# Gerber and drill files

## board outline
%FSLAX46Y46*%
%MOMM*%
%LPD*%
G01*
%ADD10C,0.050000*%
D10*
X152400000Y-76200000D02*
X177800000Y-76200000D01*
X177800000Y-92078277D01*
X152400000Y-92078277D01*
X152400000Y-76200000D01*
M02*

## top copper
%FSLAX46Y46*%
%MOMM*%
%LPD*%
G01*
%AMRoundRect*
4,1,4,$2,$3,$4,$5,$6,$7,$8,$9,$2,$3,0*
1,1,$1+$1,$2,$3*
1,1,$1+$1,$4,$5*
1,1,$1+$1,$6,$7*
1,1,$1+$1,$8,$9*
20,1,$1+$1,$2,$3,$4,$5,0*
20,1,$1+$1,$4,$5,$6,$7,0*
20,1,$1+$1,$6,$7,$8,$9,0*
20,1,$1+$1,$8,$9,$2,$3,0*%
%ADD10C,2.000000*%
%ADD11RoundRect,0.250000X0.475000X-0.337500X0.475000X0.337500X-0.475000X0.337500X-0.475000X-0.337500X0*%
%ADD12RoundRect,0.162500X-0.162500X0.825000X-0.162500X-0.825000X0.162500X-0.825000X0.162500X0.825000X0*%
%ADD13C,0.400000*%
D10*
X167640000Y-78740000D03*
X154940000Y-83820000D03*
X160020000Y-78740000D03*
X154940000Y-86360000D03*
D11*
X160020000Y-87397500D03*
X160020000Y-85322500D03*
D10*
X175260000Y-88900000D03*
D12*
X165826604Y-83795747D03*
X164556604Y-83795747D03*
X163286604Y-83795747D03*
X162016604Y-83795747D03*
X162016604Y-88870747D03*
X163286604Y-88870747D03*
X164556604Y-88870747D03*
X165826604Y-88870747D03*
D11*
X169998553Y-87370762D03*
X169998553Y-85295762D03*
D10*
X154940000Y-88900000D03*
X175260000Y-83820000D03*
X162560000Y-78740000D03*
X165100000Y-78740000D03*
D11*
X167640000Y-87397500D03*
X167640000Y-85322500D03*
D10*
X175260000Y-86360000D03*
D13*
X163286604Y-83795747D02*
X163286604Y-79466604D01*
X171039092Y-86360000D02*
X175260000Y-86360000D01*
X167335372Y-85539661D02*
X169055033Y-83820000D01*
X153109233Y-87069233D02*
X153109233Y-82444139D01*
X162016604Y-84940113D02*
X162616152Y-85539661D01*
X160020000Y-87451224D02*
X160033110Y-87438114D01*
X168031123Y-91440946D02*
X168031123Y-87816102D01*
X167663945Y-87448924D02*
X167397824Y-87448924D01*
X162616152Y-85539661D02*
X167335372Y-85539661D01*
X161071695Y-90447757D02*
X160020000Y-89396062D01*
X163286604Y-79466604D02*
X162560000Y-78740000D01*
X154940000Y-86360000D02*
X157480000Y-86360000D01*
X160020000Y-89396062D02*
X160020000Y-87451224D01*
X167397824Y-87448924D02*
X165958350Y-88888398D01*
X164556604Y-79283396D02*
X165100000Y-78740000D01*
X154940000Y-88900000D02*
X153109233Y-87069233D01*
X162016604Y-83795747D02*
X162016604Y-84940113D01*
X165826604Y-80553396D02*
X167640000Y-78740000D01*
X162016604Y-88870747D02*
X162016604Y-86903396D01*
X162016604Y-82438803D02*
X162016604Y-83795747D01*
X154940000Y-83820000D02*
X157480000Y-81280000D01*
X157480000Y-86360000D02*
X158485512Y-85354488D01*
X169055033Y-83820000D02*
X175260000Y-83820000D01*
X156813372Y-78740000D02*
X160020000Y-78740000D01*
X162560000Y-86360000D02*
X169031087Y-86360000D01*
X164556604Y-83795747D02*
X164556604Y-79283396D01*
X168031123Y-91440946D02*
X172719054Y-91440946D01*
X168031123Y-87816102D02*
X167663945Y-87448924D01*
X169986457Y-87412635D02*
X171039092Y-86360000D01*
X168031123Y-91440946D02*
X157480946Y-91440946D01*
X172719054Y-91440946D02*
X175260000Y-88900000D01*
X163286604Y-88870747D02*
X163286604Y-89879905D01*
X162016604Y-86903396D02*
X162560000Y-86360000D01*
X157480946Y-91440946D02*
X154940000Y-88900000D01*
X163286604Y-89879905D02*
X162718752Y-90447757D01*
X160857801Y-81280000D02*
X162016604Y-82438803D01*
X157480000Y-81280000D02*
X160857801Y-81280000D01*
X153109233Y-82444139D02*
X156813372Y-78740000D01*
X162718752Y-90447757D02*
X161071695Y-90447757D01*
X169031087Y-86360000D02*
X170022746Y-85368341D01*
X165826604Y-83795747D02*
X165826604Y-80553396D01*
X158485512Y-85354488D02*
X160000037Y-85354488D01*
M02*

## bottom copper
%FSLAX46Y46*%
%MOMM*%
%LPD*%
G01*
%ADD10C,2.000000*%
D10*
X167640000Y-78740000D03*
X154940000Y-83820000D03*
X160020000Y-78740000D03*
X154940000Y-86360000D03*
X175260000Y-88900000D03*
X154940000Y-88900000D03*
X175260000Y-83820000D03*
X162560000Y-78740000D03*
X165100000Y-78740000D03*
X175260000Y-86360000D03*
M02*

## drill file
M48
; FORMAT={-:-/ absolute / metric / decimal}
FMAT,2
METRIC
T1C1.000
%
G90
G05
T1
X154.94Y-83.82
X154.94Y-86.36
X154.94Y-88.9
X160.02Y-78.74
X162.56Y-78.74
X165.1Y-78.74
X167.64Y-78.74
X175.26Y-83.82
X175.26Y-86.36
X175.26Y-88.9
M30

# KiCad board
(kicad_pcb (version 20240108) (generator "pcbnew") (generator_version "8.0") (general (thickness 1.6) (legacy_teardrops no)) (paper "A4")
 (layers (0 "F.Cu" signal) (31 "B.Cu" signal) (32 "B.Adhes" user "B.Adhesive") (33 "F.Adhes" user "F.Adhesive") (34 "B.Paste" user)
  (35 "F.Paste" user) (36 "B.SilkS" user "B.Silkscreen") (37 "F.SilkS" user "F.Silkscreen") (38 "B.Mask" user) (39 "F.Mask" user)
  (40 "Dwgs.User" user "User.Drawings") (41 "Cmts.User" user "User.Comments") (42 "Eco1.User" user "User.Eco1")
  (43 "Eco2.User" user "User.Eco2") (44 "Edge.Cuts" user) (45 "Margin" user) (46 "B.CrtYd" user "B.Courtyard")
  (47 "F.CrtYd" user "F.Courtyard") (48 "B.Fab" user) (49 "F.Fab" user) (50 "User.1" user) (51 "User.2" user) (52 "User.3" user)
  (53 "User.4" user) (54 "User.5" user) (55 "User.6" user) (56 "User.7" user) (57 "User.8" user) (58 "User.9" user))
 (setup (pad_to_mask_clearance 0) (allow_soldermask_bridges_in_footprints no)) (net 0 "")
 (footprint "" (layer "F.Cu") (at 167.64 78.74)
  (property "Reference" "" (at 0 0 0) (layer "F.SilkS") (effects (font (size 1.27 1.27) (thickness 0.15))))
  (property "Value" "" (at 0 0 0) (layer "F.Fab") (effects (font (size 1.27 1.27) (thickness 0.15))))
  (pad "1" thru_hole circle (at 0 0) (size 2 2) (drill 1) (layers "*.Cu" "*.Mask") (remove_unused_layers no)))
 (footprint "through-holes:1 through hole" (layer "F.Cu") (at 154.94 83.82)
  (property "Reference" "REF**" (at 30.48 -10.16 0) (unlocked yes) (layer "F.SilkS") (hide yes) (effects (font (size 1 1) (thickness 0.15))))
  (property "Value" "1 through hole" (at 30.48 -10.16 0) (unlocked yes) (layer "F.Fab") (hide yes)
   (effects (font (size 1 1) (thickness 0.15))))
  (pad "1" thru_hole circle (at 0 0) (size 2 2) (drill 1) (layers "*.Cu" "*.Mask") (remove_unused_layers no)))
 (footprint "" (layer "F.Cu") (at 160.02 78.74)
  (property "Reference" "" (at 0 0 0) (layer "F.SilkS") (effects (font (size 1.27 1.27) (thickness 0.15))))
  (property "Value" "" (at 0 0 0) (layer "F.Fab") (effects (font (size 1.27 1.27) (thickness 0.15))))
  (pad "1" thru_hole circle (at 0 0) (size 2 2) (drill 1) (layers "*.Cu" "*.Mask") (remove_unused_layers no)))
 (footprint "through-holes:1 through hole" (layer "F.Cu") (at 154.94 86.36)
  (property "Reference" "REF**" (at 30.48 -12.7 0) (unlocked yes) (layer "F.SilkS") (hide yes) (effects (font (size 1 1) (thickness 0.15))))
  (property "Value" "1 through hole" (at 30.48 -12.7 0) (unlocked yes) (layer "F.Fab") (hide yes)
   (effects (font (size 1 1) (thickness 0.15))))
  (pad "1" thru_hole circle (at 0 0) (size 2 2) (drill 1) (layers "*.Cu" "*.Mask") (remove_unused_layers no)))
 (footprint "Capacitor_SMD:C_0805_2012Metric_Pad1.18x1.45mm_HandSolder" (layer "F.Cu") (at 160.02 86.36 90)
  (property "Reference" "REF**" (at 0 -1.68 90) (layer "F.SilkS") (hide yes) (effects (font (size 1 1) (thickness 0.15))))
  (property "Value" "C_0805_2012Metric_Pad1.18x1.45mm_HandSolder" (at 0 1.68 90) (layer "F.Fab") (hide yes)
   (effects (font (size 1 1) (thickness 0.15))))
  (pad "1" smd roundrect (at -1.0375 0 90) (size 1.175 1.45) (layers "F.Cu" "F.Paste" "F.Mask") (roundrect_rratio 0.212766))
  (pad "2" smd roundrect (at 1.0375 0 90) (size 1.175 1.45) (layers "F.Cu" "F.Paste" "F.Mask") (roundrect_rratio 0.212766)))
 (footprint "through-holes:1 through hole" (layer "F.Cu") (at 175.26 88.9)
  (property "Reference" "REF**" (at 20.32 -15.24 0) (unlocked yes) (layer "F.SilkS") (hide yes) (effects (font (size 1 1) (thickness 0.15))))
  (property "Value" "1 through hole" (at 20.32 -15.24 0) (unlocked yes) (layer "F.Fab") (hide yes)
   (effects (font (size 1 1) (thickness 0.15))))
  (pad "1" thru_hole circle (at 0 0) (size 2 2) (drill 1) (layers "*.Cu" "*.Mask") (remove_unused_layers no)))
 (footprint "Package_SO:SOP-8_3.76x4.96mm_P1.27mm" (layer "F.Cu") (at 163.921604 86.333247 -90)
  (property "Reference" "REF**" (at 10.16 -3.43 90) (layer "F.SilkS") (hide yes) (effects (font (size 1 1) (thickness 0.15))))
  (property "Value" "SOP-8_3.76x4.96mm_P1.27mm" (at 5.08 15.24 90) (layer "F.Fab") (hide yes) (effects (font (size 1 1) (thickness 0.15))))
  (pad "1" smd roundrect (at -2.5375 -1.905 270) (size 1.975 0.65) (layers "F.Cu" "F.Paste" "F.Mask") (roundrect_rratio 0.25))
  (pad "2" smd roundrect (at -2.5375 -0.635 270) (size 1.975 0.65) (layers "F.Cu" "F.Paste" "F.Mask") (roundrect_rratio 0.25))
  (pad "3" smd roundrect (at -2.5375 0.635 270) (size 1.975 0.65) (layers "F.Cu" "F.Paste" "F.Mask") (roundrect_rratio 0.25))
  (pad "4" smd roundrect (at -2.5375 1.905 270) (size 1.975 0.65) (layers "F.Cu" "F.Paste" "F.Mask") (roundrect_rratio 0.25))
  (pad "5" smd roundrect (at 2.5375 1.905 270) (size 1.975 0.65) (layers "F.Cu" "F.Paste" "F.Mask") (roundrect_rratio 0.25))
  (pad "6" smd roundrect (at 2.5375 0.635 270) (size 1.975 0.65) (layers "F.Cu" "F.Paste" "F.Mask") (roundrect_rratio 0.25))
  (pad "7" smd roundrect (at 2.5375 -0.635 270) (size 1.975 0.65) (layers "F.Cu" "F.Paste" "F.Mask") (roundrect_rratio 0.25))
  (pad "8" smd roundrect (at 2.5375 -1.905 270) (size 1.975 0.65) (layers "F.Cu" "F.Paste" "F.Mask") (roundrect_rratio 0.25)))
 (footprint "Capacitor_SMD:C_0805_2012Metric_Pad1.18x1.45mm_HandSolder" (layer "F.Cu") (at 169.998553 86.333262 90)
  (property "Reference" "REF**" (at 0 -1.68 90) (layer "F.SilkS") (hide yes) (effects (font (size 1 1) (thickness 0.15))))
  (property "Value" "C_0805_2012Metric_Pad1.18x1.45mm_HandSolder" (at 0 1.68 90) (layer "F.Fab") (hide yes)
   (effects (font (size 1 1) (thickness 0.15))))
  (pad "1" smd roundrect (at -1.0375 0 90) (size 1.175 1.45) (layers "F.Cu" "F.Paste" "F.Mask") (roundrect_rratio 0.212766))
  (pad "2" smd roundrect (at 1.0375 0 90) (size 1.175 1.45) (layers "F.Cu" "F.Paste" "F.Mask") (roundrect_rratio 0.212766)))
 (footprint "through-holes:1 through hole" (layer "F.Cu") (at 154.94 88.9)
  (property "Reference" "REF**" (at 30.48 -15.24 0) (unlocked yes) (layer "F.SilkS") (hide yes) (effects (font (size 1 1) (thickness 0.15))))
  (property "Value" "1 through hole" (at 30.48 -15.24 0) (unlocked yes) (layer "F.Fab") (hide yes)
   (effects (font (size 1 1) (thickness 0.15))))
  (pad "1" thru_hole circle (at 0 0) (size 2 2) (drill 1) (layers "*.Cu" "*.Mask") (remove_unused_layers no)))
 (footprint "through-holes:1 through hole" (layer "F.Cu") (at 175.26 83.82)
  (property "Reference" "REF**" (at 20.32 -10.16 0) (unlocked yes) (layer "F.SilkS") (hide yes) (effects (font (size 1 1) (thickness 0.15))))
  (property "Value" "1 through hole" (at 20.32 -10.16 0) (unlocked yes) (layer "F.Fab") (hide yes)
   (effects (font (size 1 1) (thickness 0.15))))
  (pad "1" thru_hole circle (at 0 0) (size 2 2) (drill 1) (layers "*.Cu" "*.Mask") (remove_unused_layers no)))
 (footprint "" (layer "F.Cu") (at 162.56 78.74)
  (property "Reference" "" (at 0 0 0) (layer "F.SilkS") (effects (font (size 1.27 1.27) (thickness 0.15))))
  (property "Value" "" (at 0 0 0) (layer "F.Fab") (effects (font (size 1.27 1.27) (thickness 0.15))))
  (pad "1" thru_hole circle (at 0 0) (size 2 2) (drill 1) (layers "*.Cu" "*.Mask") (remove_unused_layers no)))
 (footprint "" (layer "F.Cu") (at 165.1 78.74)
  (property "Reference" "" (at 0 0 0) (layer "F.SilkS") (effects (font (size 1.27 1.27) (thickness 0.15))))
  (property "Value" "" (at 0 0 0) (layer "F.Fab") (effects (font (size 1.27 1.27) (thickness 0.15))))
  (pad "1" thru_hole circle (at 0 0) (size 2 2) (drill 1) (layers "*.Cu" "*.Mask") (remove_unused_layers no)))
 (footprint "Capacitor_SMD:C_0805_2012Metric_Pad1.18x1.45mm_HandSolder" (layer "F.Cu") (at 167.64 86.36 90)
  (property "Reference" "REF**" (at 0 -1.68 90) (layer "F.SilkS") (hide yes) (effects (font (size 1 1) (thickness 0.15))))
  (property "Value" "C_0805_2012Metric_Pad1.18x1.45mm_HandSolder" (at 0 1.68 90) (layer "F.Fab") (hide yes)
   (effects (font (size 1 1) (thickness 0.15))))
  (pad "1" smd roundrect (at -1.0375 0 90) (size 1.175 1.45) (layers "F.Cu" "F.Paste" "F.Mask") (roundrect_rratio 0.212766))
  (pad "2" smd roundrect (at 1.0375 0 90) (size 1.175 1.45) (layers "F.Cu" "F.Paste" "F.Mask") (roundrect_rratio 0.212766)))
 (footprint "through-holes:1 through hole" (layer "F.Cu") (at 175.26 86.36)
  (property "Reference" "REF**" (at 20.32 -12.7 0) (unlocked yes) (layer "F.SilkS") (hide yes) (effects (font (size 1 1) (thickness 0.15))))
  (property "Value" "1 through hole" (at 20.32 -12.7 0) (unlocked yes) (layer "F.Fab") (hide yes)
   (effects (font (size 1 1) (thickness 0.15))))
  (pad "1" thru_hole circle (at 0 0) (size 2 2) (drill 1) (layers "*.Cu" "*.Mask") (remove_unused_layers no)))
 (gr_rect (start 152.4 76.2) (end 177.8 92.078277) (stroke (width 0.05) (type default)) (fill none) (layer "Edge.Cuts"))
 (segment (start 163.286604 83.795747) (end 163.286604 79.466604) (width 0.4) (layer "F.Cu") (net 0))
 (segment (start 171.039092 86.36) (end 175.26 86.36) (width 0.4) (layer "F.Cu") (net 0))
 (segment (start 167.335372 85.539661) (end 169.055033 83.82) (width 0.4) (layer "F.Cu") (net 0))
 (segment (start 153.109233 87.069233) (end 153.109233 82.444139) (width 0.4) (layer "F.Cu") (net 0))
 (segment (start 162.016604 84.940113) (end 162.616152 85.539661) (width 0.4) (layer "F.Cu") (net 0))
 (segment (start 160.02 87.451224) (end 160.03311 87.438114) (width 0.4) (layer "F.Cu") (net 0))
 (segment (start 168.031123 91.440946) (end 168.031123 87.816102) (width 0.4) (layer "F.Cu") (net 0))
 (segment (start 167.663945 87.448924) (end 167.397824 87.448924) (width 0.4) (layer "F.Cu") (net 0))
 (segment (start 162.616152 85.539661) (end 167.335372 85.539661) (width 0.4) (layer "F.Cu") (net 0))
 (segment (start 161.071695 90.447757) (end 160.02 89.396062) (width 0.4) (layer "F.Cu") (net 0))
 (segment (start 163.286604 79.466604) (end 162.56 78.74) (width 0.4) (layer "F.Cu") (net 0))
 (segment (start 154.94 86.36) (end 157.48 86.36) (width 0.4) (layer "F.Cu") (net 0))
 (segment (start 160.02 89.396062) (end 160.02 87.451224) (width 0.4) (layer "F.Cu") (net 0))
 (segment (start 167.397824 87.448924) (end 165.95835 88.888398) (width 0.4) (layer "F.Cu") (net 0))
 (segment (start 164.556604 79.283396) (end 165.1 78.74) (width 0.4) (layer "F.Cu") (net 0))
 (segment (start 154.94 88.9) (end 153.109233 87.069233) (width 0.4) (layer "F.Cu") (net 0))
 (segment (start 162.016604 83.795747) (end 162.016604 84.940113) (width 0.4) (layer "F.Cu") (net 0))
 (segment (start 165.826604 80.553396) (end 167.64 78.74) (width 0.4) (layer "F.Cu") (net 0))
 (segment (start 162.016604 88.870747) (end 162.016604 86.903396) (width 0.4) (layer "F.Cu") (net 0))
 (segment (start 162.016604 82.438803) (end 162.016604 83.795747) (width 0.4) (layer "F.Cu") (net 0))
 (segment (start 154.94 83.82) (end 157.48 81.28) (width 0.4) (layer "F.Cu") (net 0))
 (segment (start 157.48 86.36) (end 158.485512 85.354488) (width 0.4) (layer "F.Cu") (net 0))
 (segment (start 169.055033 83.82) (end 175.26 83.82) (width 0.4) (layer "F.Cu") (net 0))
 (segment (start 156.813372 78.74) (end 160.02 78.74) (width 0.4) (layer "F.Cu") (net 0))
 (segment (start 162.56 86.36) (end 169.031087 86.36) (width 0.4) (layer "F.Cu") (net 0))
 (segment (start 164.556604 83.795747) (end 164.556604 79.283396) (width 0.4) (layer "F.Cu") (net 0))
 (segment (start 168.031123 91.440946) (end 172.719054 91.440946) (width 0.4) (layer "F.Cu") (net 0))
 (segment (start 168.031123 87.816102) (end 167.663945 87.448924) (width 0.4) (layer "F.Cu") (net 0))
 (segment (start 169.986457 87.412635) (end 171.039092 86.36) (width 0.4) (layer "F.Cu") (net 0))
 (segment (start 168.031123 91.440946) (end 157.480946 91.440946) (width 0.4) (layer "F.Cu") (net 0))
 (segment (start 172.719054 91.440946) (end 175.26 88.9) (width 0.4) (layer "F.Cu") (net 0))
 (segment (start 163.286604 88.870747) (end 163.286604 89.879905) (width 0.4) (layer "F.Cu") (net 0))
 (segment (start 162.016604 86.903396) (end 162.56 86.36) (width 0.4) (layer "F.Cu") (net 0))
 (segment (start 157.480946 91.440946) (end 154.94 88.9) (width 0.4) (layer "F.Cu") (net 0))
 (segment (start 163.286604 89.879905) (end 162.718752 90.447757) (width 0.4) (layer "F.Cu") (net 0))
 (segment (start 160.857801 81.28) (end 162.016604 82.438803) (width 0.4) (layer "F.Cu") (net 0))
 (segment (start 157.48 81.28) (end 160.857801 81.28) (width 0.4) (layer "F.Cu") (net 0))
 (segment (start 153.109233 82.444139) (end 156.813372 78.74) (width 0.4) (layer "F.Cu") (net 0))
 (segment (start 162.718752 90.447757) (end 161.071695 90.447757) (width 0.4) (layer "F.Cu") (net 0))
 (segment (start 169.031087 86.36) (end 170.022746 85.368341) (width 0.4) (layer "F.Cu") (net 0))
 (segment (start 165.826604 83.795747) (end 165.826604 80.553396) (width 0.4) (layer "F.Cu") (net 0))
 (segment (start 158.485512 85.354488) (end 160.000037 85.354488) (width 0.4) (layer "F.Cu") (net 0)))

